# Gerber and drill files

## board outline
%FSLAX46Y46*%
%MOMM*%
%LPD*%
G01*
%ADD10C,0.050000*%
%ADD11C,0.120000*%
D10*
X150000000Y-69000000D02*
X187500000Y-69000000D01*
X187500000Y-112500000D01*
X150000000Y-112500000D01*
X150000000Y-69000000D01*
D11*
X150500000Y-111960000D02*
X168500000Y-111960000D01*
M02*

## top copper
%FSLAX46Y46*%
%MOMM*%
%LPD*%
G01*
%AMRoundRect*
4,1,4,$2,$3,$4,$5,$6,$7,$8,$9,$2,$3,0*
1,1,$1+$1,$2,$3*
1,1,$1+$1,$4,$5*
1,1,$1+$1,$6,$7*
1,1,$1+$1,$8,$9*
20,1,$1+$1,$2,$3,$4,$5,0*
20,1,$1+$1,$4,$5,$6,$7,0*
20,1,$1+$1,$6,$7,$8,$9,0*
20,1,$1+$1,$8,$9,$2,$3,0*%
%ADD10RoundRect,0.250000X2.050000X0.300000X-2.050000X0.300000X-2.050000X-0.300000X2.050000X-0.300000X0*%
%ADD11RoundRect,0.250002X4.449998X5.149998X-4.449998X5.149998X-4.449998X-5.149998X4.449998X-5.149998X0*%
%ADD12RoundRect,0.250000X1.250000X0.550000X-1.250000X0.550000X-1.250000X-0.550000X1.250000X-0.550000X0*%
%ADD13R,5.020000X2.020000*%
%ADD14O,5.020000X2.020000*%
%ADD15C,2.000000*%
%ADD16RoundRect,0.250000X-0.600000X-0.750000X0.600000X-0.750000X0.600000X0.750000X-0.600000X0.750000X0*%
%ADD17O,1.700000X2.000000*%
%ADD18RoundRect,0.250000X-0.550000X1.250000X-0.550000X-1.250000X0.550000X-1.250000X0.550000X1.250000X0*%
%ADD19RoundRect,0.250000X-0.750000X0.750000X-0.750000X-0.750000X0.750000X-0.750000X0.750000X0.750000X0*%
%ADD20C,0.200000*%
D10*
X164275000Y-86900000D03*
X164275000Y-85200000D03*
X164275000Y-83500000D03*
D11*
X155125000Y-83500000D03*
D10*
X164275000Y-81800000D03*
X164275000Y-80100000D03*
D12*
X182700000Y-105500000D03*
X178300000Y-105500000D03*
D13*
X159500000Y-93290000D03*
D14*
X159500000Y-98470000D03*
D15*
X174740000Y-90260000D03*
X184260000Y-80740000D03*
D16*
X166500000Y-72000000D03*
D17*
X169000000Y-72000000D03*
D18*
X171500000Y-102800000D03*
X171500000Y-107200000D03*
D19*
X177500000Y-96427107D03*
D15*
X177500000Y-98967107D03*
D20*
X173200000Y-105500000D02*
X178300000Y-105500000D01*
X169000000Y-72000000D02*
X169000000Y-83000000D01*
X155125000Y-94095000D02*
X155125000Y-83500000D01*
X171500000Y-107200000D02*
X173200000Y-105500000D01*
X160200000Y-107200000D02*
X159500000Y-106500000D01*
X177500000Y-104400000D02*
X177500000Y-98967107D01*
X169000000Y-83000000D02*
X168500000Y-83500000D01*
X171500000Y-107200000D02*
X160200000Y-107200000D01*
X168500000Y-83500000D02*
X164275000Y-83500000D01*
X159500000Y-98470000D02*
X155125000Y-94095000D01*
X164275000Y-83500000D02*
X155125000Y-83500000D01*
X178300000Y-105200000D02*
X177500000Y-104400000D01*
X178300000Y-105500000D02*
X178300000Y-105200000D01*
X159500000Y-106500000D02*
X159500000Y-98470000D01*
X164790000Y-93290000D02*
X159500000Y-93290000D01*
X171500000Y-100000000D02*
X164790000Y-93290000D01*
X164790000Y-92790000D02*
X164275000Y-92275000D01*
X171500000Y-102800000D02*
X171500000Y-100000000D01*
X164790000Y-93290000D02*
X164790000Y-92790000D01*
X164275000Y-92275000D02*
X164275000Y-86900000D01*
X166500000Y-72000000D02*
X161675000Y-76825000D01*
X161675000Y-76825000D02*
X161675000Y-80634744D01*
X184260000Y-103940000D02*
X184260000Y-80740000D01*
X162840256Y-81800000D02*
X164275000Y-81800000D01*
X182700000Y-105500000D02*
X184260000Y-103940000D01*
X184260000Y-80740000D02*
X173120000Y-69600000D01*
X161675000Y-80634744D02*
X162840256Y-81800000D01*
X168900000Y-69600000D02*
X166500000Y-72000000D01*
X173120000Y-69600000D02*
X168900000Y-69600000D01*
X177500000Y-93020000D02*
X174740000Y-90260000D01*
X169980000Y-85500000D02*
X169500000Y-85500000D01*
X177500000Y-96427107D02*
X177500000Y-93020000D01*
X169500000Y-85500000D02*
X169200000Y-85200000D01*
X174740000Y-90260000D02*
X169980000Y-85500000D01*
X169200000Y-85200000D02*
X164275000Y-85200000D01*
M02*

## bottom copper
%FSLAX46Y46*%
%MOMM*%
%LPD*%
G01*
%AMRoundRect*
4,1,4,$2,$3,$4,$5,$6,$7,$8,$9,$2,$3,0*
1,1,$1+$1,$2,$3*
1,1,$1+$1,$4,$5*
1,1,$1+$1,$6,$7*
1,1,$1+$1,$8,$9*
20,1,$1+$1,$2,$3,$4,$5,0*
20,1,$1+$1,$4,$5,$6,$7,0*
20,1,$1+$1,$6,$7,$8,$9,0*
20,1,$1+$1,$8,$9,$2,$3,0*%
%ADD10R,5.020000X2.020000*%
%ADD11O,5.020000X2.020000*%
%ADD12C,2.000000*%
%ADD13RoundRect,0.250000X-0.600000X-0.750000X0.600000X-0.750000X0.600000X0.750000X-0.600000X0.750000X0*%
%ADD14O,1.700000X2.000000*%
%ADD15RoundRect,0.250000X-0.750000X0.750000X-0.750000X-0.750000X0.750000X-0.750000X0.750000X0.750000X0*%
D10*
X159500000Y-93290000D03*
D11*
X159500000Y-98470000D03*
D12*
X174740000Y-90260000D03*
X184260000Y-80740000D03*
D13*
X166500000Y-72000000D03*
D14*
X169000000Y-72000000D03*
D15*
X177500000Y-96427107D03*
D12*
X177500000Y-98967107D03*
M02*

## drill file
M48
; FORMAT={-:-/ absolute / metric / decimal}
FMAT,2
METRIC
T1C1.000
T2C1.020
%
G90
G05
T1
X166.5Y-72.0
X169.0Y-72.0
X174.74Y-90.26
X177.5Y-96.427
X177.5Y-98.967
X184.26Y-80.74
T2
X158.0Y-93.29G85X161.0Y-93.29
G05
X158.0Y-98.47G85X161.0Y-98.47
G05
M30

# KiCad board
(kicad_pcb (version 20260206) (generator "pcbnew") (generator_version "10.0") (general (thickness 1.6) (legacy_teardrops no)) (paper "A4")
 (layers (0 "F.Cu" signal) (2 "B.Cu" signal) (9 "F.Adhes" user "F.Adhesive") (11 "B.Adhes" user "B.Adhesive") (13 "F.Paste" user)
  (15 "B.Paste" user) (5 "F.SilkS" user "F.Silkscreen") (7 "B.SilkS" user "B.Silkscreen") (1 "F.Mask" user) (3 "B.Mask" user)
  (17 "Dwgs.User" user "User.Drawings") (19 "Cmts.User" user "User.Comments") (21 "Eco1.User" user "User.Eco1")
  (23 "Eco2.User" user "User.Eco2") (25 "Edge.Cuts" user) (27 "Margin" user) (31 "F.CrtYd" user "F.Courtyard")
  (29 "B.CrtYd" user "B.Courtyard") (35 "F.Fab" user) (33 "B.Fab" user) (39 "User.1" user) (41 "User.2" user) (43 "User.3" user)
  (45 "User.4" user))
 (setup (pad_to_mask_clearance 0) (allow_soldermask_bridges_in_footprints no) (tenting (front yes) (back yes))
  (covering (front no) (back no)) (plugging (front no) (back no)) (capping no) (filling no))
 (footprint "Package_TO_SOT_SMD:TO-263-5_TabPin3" (layer "F.Cu") (at 156.625 83.5 180)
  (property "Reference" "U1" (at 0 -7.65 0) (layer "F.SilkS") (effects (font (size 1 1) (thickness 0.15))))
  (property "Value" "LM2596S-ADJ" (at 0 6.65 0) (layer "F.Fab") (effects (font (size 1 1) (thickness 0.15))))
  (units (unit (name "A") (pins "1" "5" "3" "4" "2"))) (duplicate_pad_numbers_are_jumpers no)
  (pad "" smd roundrect (at -0.925 -2.775 180) (size 4.55 5.25) (layers "F.Paste") (roundrect_rratio 0.054945))
  (pad "" smd roundrect (at -0.925 2.775 180) (size 4.55 5.25) (layers "F.Paste") (roundrect_rratio 0.054945))
  (pad "" smd roundrect (at 3.925 -2.775 180) (size 4.55 5.25) (layers "F.Paste") (roundrect_rratio 0.054945))
  (pad "" smd roundrect (at 3.925 2.775 180) (size 4.55 5.25) (layers "F.Paste") (roundrect_rratio 0.054945))
  (pad "1" smd roundrect (at -7.65 -3.4 180) (size 4.6 1.1) (layers "F.Cu" "F.Mask" "F.Paste") (roundrect_rratio 0.227273)
   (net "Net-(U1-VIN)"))
  (pad "2" smd roundrect (at -7.65 -1.7 180) (size 4.6 1.1) (layers "F.Cu" "F.Mask" "F.Paste") (roundrect_rratio 0.227273)
   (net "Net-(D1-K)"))
  (pad "3" smd roundrect (at -7.65 0 180) (size 4.6 1.1) (layers "F.Cu" "F.Mask" "F.Paste") (roundrect_rratio 0.227273) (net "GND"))
  (pad "3" smd roundrect (at 1.5 0 180) (size 9.4 10.8) (layers "F.Cu" "F.Mask") (roundrect_rratio 0.026596) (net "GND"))
  (pad "4" smd roundrect (at -7.65 1.7 180) (size 4.6 1.1) (layers "F.Cu" "F.Mask" "F.Paste") (roundrect_rratio 0.227273)
   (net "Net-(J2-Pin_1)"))
  (pad "5" smd roundrect (at -7.65 3.4 180) (size 4.6 1.1) (layers "F.Cu" "F.Mask" "F.Paste") (roundrect_rratio 0.227273)
   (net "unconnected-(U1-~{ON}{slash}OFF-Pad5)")))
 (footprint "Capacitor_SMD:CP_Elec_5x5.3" (layer "F.Cu") (at 180.5 105.5 180)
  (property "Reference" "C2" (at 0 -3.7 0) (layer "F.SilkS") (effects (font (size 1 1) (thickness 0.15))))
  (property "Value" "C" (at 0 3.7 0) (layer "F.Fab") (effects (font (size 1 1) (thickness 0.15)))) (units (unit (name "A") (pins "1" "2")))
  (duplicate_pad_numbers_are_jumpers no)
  (pad "1" smd roundrect (at -2.2 0 180) (size 3 1.6) (layers "F.Cu" "F.Mask" "F.Paste") (roundrect_rratio 0.15625) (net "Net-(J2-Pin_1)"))
  (pad "2" smd roundrect (at 2.2 0 180) (size 3 1.6) (layers "F.Cu" "F.Mask" "F.Paste") (roundrect_rratio 0.15625) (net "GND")))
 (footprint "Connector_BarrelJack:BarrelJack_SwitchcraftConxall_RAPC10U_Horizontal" (layer "F.Cu") (at 159.5 93.29 90)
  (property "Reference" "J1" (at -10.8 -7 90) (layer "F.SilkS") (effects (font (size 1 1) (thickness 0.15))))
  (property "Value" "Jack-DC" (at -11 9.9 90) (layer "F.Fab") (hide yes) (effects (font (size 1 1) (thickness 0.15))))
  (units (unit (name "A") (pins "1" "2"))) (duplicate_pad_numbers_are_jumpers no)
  (fp_line (start -18.67 -9) (end -18.67 9) (stroke (width 0.12) (type solid)) (layer "Edge.Cuts"))
  (pad "1" thru_hole rect (at 0 0 90) (size 2.02 5.02) (drill oval 1.02 4.02) (layers "*.Cu" "*.Mask") (remove_unused_layers no)
   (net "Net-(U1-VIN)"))
  (pad "2" thru_hole oval (at -5.18 0 90) (size 2.02 5.02) (drill oval 1.02 4.02) (layers "*.Cu" "*.Mask") (remove_unused_layers no)
   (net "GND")))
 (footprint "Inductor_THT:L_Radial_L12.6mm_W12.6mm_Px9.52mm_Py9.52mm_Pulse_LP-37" (layer "F.Cu") (at 174.74 90.26)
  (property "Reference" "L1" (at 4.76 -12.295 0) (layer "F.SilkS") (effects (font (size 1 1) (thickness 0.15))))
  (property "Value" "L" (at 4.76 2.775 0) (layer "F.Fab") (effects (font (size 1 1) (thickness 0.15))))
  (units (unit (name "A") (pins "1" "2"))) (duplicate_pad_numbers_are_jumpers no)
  (pad "1" thru_hole circle (at 0 0) (size 2 2) (drill 1) (layers "*.Cu" "*.Mask") (remove_unused_layers no) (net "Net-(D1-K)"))
  (pad "2" thru_hole circle (at 9.52 -9.52) (size 2 2) (drill 1) (layers "*.Cu" "*.Mask") (remove_unused_layers no) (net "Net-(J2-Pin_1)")))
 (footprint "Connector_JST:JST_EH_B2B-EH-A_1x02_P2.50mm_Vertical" (layer "F.Cu") (at 166.5 72)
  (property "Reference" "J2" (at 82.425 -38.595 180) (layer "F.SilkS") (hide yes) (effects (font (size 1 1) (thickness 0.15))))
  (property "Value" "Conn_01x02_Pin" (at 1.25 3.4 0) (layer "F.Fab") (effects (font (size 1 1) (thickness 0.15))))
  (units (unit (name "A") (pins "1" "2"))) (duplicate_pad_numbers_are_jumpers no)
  (pad "1" thru_hole roundrect (at 0 0) (size 1.7 2) (drill 1) (layers "*.Cu" "*.Mask") (remove_unused_layers no)
   (roundrect_rratio 0.147059) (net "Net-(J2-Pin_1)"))
  (pad "2" thru_hole oval (at 2.5 0) (size 1.7 2) (drill 1) (layers "*.Cu" "*.Mask") (remove_unused_layers no) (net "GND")))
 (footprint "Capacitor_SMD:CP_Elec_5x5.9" (layer "F.Cu") (at 171.5 105 -90)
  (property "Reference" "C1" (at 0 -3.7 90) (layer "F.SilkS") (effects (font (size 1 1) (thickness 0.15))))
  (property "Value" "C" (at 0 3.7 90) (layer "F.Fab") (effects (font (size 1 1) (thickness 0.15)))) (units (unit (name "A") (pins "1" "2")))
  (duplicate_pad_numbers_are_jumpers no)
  (pad "1" smd roundrect (at -2.2 0 270) (size 3 1.6) (layers "F.Cu" "F.Mask" "F.Paste") (roundrect_rratio 0.15625) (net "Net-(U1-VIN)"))
  (pad "2" smd roundrect (at 2.2 0 270) (size 3 1.6) (layers "F.Cu" "F.Mask" "F.Paste") (roundrect_rratio 0.15625) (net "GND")))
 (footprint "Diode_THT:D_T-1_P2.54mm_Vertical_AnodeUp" (layer "F.Cu") (at 177.5 96.427107 -90)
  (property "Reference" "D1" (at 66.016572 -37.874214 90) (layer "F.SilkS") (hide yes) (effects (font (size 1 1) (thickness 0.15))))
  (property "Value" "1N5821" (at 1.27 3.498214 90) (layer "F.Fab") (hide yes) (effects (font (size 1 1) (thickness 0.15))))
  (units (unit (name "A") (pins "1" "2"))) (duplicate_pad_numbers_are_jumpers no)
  (pad "1" thru_hole roundrect (at 0 0 270) (size 2 2) (drill 1) (layers "*.Cu" "*.Mask") (remove_unused_layers no) (roundrect_rratio 0.125)
   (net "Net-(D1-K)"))
  (pad "2" thru_hole circle (at 2.54 0 270) (size 2 2) (drill 1) (layers "*.Cu" "*.Mask") (remove_unused_layers no) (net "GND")))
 (gr_rect (start 150 69) (end 187.5 112.5) (stroke (width 0.05) (type default)) (fill no) (layer "Edge.Cuts"))
 (segment (start 173.2 105.5) (end 178.3 105.5) (width 0.2) (layer "F.Cu") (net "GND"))
 (segment (start 169 72) (end 169 83) (width 0.2) (layer "F.Cu") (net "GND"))
 (segment (start 155.125 94.095) (end 155.125 83.5) (width 0.2) (layer "F.Cu") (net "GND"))
 (segment (start 171.5 107.2) (end 173.2 105.5) (width 0.2) (layer "F.Cu") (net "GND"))
 (segment (start 160.2 107.2) (end 159.5 106.5) (width 0.2) (layer "F.Cu") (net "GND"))
 (segment (start 177.5 104.4) (end 177.5 98.967107) (width 0.2) (layer "F.Cu") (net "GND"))
 (segment (start 169 83) (end 168.5 83.5) (width 0.2) (layer "F.Cu") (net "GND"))
 (segment (start 171.5 107.2) (end 160.2 107.2) (width 0.2) (layer "F.Cu") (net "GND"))
 (segment (start 168.5 83.5) (end 164.275 83.5) (width 0.2) (layer "F.Cu") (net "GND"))
 (segment (start 159.5 98.47) (end 155.125 94.095) (width 0.2) (layer "F.Cu") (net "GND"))
 (segment (start 164.275 83.5) (end 155.125 83.5) (width 0.2) (layer "F.Cu") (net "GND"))
 (segment (start 178.3 105.2) (end 177.5 104.4) (width 0.2) (layer "F.Cu") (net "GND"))
 (segment (start 178.3 105.5) (end 178.3 105.2) (width 0.2) (layer "F.Cu") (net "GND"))
 (segment (start 159.5 106.5) (end 159.5 98.47) (width 0.2) (layer "F.Cu") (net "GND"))
 (segment (start 164.79 93.29) (end 159.5 93.29) (width 0.2) (layer "F.Cu") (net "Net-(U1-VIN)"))
 (segment (start 171.5 100) (end 164.79 93.29) (width 0.2) (layer "F.Cu") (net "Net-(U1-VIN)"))
 (segment (start 164.79 92.79) (end 164.275 92.275) (width 0.2) (layer "F.Cu") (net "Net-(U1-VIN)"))
 (segment (start 171.5 102.8) (end 171.5 100) (width 0.2) (layer "F.Cu") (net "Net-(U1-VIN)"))
 (segment (start 164.79 93.29) (end 164.79 92.79) (width 0.2) (layer "F.Cu") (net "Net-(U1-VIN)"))
 (segment (start 164.275 92.275) (end 164.275 86.9) (width 0.2) (layer "F.Cu") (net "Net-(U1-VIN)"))
 (segment (start 166.5 72) (end 161.675 76.825) (width 0.2) (layer "F.Cu") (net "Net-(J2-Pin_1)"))
 (segment (start 161.675 76.825) (end 161.675 80.634744) (width 0.2) (layer "F.Cu") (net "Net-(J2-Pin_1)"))
 (segment (start 184.26 103.94) (end 184.26 80.74) (width 0.2) (layer "F.Cu") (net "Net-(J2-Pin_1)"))
 (segment (start 162.840256 81.8) (end 164.275 81.8) (width 0.2) (layer "F.Cu") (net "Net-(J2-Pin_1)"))
 (segment (start 182.7 105.5) (end 184.26 103.94) (width 0.2) (layer "F.Cu") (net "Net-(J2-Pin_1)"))
 (segment (start 184.26 80.74) (end 173.12 69.6) (width 0.2) (layer "F.Cu") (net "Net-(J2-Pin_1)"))
 (segment (start 161.675 80.634744) (end 162.840256 81.8) (width 0.2) (layer "F.Cu") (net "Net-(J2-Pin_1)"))
 (segment (start 168.9 69.6) (end 166.5 72) (width 0.2) (layer "F.Cu") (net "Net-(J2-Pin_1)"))
 (segment (start 173.12 69.6) (end 168.9 69.6) (width 0.2) (layer "F.Cu") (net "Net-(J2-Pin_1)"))
 (segment (start 177.5 93.02) (end 174.74 90.26) (width 0.2) (layer "F.Cu") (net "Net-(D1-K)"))
 (segment (start 169.98 85.5) (end 169.5 85.5) (width 0.2) (layer "F.Cu") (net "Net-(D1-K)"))
 (segment (start 177.5 96.427107) (end 177.5 93.02) (width 0.2) (layer "F.Cu") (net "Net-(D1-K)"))
 (segment (start 169.5 85.5) (end 169.2 85.2) (width 0.2) (layer "F.Cu") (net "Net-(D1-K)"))
 (segment (start 174.74 90.26) (end 169.98 85.5) (width 0.2) (layer "F.Cu") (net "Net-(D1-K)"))
 (segment (start 169.2 85.2) (end 164.275 85.2) (width 0.2) (layer "F.Cu") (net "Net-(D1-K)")))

